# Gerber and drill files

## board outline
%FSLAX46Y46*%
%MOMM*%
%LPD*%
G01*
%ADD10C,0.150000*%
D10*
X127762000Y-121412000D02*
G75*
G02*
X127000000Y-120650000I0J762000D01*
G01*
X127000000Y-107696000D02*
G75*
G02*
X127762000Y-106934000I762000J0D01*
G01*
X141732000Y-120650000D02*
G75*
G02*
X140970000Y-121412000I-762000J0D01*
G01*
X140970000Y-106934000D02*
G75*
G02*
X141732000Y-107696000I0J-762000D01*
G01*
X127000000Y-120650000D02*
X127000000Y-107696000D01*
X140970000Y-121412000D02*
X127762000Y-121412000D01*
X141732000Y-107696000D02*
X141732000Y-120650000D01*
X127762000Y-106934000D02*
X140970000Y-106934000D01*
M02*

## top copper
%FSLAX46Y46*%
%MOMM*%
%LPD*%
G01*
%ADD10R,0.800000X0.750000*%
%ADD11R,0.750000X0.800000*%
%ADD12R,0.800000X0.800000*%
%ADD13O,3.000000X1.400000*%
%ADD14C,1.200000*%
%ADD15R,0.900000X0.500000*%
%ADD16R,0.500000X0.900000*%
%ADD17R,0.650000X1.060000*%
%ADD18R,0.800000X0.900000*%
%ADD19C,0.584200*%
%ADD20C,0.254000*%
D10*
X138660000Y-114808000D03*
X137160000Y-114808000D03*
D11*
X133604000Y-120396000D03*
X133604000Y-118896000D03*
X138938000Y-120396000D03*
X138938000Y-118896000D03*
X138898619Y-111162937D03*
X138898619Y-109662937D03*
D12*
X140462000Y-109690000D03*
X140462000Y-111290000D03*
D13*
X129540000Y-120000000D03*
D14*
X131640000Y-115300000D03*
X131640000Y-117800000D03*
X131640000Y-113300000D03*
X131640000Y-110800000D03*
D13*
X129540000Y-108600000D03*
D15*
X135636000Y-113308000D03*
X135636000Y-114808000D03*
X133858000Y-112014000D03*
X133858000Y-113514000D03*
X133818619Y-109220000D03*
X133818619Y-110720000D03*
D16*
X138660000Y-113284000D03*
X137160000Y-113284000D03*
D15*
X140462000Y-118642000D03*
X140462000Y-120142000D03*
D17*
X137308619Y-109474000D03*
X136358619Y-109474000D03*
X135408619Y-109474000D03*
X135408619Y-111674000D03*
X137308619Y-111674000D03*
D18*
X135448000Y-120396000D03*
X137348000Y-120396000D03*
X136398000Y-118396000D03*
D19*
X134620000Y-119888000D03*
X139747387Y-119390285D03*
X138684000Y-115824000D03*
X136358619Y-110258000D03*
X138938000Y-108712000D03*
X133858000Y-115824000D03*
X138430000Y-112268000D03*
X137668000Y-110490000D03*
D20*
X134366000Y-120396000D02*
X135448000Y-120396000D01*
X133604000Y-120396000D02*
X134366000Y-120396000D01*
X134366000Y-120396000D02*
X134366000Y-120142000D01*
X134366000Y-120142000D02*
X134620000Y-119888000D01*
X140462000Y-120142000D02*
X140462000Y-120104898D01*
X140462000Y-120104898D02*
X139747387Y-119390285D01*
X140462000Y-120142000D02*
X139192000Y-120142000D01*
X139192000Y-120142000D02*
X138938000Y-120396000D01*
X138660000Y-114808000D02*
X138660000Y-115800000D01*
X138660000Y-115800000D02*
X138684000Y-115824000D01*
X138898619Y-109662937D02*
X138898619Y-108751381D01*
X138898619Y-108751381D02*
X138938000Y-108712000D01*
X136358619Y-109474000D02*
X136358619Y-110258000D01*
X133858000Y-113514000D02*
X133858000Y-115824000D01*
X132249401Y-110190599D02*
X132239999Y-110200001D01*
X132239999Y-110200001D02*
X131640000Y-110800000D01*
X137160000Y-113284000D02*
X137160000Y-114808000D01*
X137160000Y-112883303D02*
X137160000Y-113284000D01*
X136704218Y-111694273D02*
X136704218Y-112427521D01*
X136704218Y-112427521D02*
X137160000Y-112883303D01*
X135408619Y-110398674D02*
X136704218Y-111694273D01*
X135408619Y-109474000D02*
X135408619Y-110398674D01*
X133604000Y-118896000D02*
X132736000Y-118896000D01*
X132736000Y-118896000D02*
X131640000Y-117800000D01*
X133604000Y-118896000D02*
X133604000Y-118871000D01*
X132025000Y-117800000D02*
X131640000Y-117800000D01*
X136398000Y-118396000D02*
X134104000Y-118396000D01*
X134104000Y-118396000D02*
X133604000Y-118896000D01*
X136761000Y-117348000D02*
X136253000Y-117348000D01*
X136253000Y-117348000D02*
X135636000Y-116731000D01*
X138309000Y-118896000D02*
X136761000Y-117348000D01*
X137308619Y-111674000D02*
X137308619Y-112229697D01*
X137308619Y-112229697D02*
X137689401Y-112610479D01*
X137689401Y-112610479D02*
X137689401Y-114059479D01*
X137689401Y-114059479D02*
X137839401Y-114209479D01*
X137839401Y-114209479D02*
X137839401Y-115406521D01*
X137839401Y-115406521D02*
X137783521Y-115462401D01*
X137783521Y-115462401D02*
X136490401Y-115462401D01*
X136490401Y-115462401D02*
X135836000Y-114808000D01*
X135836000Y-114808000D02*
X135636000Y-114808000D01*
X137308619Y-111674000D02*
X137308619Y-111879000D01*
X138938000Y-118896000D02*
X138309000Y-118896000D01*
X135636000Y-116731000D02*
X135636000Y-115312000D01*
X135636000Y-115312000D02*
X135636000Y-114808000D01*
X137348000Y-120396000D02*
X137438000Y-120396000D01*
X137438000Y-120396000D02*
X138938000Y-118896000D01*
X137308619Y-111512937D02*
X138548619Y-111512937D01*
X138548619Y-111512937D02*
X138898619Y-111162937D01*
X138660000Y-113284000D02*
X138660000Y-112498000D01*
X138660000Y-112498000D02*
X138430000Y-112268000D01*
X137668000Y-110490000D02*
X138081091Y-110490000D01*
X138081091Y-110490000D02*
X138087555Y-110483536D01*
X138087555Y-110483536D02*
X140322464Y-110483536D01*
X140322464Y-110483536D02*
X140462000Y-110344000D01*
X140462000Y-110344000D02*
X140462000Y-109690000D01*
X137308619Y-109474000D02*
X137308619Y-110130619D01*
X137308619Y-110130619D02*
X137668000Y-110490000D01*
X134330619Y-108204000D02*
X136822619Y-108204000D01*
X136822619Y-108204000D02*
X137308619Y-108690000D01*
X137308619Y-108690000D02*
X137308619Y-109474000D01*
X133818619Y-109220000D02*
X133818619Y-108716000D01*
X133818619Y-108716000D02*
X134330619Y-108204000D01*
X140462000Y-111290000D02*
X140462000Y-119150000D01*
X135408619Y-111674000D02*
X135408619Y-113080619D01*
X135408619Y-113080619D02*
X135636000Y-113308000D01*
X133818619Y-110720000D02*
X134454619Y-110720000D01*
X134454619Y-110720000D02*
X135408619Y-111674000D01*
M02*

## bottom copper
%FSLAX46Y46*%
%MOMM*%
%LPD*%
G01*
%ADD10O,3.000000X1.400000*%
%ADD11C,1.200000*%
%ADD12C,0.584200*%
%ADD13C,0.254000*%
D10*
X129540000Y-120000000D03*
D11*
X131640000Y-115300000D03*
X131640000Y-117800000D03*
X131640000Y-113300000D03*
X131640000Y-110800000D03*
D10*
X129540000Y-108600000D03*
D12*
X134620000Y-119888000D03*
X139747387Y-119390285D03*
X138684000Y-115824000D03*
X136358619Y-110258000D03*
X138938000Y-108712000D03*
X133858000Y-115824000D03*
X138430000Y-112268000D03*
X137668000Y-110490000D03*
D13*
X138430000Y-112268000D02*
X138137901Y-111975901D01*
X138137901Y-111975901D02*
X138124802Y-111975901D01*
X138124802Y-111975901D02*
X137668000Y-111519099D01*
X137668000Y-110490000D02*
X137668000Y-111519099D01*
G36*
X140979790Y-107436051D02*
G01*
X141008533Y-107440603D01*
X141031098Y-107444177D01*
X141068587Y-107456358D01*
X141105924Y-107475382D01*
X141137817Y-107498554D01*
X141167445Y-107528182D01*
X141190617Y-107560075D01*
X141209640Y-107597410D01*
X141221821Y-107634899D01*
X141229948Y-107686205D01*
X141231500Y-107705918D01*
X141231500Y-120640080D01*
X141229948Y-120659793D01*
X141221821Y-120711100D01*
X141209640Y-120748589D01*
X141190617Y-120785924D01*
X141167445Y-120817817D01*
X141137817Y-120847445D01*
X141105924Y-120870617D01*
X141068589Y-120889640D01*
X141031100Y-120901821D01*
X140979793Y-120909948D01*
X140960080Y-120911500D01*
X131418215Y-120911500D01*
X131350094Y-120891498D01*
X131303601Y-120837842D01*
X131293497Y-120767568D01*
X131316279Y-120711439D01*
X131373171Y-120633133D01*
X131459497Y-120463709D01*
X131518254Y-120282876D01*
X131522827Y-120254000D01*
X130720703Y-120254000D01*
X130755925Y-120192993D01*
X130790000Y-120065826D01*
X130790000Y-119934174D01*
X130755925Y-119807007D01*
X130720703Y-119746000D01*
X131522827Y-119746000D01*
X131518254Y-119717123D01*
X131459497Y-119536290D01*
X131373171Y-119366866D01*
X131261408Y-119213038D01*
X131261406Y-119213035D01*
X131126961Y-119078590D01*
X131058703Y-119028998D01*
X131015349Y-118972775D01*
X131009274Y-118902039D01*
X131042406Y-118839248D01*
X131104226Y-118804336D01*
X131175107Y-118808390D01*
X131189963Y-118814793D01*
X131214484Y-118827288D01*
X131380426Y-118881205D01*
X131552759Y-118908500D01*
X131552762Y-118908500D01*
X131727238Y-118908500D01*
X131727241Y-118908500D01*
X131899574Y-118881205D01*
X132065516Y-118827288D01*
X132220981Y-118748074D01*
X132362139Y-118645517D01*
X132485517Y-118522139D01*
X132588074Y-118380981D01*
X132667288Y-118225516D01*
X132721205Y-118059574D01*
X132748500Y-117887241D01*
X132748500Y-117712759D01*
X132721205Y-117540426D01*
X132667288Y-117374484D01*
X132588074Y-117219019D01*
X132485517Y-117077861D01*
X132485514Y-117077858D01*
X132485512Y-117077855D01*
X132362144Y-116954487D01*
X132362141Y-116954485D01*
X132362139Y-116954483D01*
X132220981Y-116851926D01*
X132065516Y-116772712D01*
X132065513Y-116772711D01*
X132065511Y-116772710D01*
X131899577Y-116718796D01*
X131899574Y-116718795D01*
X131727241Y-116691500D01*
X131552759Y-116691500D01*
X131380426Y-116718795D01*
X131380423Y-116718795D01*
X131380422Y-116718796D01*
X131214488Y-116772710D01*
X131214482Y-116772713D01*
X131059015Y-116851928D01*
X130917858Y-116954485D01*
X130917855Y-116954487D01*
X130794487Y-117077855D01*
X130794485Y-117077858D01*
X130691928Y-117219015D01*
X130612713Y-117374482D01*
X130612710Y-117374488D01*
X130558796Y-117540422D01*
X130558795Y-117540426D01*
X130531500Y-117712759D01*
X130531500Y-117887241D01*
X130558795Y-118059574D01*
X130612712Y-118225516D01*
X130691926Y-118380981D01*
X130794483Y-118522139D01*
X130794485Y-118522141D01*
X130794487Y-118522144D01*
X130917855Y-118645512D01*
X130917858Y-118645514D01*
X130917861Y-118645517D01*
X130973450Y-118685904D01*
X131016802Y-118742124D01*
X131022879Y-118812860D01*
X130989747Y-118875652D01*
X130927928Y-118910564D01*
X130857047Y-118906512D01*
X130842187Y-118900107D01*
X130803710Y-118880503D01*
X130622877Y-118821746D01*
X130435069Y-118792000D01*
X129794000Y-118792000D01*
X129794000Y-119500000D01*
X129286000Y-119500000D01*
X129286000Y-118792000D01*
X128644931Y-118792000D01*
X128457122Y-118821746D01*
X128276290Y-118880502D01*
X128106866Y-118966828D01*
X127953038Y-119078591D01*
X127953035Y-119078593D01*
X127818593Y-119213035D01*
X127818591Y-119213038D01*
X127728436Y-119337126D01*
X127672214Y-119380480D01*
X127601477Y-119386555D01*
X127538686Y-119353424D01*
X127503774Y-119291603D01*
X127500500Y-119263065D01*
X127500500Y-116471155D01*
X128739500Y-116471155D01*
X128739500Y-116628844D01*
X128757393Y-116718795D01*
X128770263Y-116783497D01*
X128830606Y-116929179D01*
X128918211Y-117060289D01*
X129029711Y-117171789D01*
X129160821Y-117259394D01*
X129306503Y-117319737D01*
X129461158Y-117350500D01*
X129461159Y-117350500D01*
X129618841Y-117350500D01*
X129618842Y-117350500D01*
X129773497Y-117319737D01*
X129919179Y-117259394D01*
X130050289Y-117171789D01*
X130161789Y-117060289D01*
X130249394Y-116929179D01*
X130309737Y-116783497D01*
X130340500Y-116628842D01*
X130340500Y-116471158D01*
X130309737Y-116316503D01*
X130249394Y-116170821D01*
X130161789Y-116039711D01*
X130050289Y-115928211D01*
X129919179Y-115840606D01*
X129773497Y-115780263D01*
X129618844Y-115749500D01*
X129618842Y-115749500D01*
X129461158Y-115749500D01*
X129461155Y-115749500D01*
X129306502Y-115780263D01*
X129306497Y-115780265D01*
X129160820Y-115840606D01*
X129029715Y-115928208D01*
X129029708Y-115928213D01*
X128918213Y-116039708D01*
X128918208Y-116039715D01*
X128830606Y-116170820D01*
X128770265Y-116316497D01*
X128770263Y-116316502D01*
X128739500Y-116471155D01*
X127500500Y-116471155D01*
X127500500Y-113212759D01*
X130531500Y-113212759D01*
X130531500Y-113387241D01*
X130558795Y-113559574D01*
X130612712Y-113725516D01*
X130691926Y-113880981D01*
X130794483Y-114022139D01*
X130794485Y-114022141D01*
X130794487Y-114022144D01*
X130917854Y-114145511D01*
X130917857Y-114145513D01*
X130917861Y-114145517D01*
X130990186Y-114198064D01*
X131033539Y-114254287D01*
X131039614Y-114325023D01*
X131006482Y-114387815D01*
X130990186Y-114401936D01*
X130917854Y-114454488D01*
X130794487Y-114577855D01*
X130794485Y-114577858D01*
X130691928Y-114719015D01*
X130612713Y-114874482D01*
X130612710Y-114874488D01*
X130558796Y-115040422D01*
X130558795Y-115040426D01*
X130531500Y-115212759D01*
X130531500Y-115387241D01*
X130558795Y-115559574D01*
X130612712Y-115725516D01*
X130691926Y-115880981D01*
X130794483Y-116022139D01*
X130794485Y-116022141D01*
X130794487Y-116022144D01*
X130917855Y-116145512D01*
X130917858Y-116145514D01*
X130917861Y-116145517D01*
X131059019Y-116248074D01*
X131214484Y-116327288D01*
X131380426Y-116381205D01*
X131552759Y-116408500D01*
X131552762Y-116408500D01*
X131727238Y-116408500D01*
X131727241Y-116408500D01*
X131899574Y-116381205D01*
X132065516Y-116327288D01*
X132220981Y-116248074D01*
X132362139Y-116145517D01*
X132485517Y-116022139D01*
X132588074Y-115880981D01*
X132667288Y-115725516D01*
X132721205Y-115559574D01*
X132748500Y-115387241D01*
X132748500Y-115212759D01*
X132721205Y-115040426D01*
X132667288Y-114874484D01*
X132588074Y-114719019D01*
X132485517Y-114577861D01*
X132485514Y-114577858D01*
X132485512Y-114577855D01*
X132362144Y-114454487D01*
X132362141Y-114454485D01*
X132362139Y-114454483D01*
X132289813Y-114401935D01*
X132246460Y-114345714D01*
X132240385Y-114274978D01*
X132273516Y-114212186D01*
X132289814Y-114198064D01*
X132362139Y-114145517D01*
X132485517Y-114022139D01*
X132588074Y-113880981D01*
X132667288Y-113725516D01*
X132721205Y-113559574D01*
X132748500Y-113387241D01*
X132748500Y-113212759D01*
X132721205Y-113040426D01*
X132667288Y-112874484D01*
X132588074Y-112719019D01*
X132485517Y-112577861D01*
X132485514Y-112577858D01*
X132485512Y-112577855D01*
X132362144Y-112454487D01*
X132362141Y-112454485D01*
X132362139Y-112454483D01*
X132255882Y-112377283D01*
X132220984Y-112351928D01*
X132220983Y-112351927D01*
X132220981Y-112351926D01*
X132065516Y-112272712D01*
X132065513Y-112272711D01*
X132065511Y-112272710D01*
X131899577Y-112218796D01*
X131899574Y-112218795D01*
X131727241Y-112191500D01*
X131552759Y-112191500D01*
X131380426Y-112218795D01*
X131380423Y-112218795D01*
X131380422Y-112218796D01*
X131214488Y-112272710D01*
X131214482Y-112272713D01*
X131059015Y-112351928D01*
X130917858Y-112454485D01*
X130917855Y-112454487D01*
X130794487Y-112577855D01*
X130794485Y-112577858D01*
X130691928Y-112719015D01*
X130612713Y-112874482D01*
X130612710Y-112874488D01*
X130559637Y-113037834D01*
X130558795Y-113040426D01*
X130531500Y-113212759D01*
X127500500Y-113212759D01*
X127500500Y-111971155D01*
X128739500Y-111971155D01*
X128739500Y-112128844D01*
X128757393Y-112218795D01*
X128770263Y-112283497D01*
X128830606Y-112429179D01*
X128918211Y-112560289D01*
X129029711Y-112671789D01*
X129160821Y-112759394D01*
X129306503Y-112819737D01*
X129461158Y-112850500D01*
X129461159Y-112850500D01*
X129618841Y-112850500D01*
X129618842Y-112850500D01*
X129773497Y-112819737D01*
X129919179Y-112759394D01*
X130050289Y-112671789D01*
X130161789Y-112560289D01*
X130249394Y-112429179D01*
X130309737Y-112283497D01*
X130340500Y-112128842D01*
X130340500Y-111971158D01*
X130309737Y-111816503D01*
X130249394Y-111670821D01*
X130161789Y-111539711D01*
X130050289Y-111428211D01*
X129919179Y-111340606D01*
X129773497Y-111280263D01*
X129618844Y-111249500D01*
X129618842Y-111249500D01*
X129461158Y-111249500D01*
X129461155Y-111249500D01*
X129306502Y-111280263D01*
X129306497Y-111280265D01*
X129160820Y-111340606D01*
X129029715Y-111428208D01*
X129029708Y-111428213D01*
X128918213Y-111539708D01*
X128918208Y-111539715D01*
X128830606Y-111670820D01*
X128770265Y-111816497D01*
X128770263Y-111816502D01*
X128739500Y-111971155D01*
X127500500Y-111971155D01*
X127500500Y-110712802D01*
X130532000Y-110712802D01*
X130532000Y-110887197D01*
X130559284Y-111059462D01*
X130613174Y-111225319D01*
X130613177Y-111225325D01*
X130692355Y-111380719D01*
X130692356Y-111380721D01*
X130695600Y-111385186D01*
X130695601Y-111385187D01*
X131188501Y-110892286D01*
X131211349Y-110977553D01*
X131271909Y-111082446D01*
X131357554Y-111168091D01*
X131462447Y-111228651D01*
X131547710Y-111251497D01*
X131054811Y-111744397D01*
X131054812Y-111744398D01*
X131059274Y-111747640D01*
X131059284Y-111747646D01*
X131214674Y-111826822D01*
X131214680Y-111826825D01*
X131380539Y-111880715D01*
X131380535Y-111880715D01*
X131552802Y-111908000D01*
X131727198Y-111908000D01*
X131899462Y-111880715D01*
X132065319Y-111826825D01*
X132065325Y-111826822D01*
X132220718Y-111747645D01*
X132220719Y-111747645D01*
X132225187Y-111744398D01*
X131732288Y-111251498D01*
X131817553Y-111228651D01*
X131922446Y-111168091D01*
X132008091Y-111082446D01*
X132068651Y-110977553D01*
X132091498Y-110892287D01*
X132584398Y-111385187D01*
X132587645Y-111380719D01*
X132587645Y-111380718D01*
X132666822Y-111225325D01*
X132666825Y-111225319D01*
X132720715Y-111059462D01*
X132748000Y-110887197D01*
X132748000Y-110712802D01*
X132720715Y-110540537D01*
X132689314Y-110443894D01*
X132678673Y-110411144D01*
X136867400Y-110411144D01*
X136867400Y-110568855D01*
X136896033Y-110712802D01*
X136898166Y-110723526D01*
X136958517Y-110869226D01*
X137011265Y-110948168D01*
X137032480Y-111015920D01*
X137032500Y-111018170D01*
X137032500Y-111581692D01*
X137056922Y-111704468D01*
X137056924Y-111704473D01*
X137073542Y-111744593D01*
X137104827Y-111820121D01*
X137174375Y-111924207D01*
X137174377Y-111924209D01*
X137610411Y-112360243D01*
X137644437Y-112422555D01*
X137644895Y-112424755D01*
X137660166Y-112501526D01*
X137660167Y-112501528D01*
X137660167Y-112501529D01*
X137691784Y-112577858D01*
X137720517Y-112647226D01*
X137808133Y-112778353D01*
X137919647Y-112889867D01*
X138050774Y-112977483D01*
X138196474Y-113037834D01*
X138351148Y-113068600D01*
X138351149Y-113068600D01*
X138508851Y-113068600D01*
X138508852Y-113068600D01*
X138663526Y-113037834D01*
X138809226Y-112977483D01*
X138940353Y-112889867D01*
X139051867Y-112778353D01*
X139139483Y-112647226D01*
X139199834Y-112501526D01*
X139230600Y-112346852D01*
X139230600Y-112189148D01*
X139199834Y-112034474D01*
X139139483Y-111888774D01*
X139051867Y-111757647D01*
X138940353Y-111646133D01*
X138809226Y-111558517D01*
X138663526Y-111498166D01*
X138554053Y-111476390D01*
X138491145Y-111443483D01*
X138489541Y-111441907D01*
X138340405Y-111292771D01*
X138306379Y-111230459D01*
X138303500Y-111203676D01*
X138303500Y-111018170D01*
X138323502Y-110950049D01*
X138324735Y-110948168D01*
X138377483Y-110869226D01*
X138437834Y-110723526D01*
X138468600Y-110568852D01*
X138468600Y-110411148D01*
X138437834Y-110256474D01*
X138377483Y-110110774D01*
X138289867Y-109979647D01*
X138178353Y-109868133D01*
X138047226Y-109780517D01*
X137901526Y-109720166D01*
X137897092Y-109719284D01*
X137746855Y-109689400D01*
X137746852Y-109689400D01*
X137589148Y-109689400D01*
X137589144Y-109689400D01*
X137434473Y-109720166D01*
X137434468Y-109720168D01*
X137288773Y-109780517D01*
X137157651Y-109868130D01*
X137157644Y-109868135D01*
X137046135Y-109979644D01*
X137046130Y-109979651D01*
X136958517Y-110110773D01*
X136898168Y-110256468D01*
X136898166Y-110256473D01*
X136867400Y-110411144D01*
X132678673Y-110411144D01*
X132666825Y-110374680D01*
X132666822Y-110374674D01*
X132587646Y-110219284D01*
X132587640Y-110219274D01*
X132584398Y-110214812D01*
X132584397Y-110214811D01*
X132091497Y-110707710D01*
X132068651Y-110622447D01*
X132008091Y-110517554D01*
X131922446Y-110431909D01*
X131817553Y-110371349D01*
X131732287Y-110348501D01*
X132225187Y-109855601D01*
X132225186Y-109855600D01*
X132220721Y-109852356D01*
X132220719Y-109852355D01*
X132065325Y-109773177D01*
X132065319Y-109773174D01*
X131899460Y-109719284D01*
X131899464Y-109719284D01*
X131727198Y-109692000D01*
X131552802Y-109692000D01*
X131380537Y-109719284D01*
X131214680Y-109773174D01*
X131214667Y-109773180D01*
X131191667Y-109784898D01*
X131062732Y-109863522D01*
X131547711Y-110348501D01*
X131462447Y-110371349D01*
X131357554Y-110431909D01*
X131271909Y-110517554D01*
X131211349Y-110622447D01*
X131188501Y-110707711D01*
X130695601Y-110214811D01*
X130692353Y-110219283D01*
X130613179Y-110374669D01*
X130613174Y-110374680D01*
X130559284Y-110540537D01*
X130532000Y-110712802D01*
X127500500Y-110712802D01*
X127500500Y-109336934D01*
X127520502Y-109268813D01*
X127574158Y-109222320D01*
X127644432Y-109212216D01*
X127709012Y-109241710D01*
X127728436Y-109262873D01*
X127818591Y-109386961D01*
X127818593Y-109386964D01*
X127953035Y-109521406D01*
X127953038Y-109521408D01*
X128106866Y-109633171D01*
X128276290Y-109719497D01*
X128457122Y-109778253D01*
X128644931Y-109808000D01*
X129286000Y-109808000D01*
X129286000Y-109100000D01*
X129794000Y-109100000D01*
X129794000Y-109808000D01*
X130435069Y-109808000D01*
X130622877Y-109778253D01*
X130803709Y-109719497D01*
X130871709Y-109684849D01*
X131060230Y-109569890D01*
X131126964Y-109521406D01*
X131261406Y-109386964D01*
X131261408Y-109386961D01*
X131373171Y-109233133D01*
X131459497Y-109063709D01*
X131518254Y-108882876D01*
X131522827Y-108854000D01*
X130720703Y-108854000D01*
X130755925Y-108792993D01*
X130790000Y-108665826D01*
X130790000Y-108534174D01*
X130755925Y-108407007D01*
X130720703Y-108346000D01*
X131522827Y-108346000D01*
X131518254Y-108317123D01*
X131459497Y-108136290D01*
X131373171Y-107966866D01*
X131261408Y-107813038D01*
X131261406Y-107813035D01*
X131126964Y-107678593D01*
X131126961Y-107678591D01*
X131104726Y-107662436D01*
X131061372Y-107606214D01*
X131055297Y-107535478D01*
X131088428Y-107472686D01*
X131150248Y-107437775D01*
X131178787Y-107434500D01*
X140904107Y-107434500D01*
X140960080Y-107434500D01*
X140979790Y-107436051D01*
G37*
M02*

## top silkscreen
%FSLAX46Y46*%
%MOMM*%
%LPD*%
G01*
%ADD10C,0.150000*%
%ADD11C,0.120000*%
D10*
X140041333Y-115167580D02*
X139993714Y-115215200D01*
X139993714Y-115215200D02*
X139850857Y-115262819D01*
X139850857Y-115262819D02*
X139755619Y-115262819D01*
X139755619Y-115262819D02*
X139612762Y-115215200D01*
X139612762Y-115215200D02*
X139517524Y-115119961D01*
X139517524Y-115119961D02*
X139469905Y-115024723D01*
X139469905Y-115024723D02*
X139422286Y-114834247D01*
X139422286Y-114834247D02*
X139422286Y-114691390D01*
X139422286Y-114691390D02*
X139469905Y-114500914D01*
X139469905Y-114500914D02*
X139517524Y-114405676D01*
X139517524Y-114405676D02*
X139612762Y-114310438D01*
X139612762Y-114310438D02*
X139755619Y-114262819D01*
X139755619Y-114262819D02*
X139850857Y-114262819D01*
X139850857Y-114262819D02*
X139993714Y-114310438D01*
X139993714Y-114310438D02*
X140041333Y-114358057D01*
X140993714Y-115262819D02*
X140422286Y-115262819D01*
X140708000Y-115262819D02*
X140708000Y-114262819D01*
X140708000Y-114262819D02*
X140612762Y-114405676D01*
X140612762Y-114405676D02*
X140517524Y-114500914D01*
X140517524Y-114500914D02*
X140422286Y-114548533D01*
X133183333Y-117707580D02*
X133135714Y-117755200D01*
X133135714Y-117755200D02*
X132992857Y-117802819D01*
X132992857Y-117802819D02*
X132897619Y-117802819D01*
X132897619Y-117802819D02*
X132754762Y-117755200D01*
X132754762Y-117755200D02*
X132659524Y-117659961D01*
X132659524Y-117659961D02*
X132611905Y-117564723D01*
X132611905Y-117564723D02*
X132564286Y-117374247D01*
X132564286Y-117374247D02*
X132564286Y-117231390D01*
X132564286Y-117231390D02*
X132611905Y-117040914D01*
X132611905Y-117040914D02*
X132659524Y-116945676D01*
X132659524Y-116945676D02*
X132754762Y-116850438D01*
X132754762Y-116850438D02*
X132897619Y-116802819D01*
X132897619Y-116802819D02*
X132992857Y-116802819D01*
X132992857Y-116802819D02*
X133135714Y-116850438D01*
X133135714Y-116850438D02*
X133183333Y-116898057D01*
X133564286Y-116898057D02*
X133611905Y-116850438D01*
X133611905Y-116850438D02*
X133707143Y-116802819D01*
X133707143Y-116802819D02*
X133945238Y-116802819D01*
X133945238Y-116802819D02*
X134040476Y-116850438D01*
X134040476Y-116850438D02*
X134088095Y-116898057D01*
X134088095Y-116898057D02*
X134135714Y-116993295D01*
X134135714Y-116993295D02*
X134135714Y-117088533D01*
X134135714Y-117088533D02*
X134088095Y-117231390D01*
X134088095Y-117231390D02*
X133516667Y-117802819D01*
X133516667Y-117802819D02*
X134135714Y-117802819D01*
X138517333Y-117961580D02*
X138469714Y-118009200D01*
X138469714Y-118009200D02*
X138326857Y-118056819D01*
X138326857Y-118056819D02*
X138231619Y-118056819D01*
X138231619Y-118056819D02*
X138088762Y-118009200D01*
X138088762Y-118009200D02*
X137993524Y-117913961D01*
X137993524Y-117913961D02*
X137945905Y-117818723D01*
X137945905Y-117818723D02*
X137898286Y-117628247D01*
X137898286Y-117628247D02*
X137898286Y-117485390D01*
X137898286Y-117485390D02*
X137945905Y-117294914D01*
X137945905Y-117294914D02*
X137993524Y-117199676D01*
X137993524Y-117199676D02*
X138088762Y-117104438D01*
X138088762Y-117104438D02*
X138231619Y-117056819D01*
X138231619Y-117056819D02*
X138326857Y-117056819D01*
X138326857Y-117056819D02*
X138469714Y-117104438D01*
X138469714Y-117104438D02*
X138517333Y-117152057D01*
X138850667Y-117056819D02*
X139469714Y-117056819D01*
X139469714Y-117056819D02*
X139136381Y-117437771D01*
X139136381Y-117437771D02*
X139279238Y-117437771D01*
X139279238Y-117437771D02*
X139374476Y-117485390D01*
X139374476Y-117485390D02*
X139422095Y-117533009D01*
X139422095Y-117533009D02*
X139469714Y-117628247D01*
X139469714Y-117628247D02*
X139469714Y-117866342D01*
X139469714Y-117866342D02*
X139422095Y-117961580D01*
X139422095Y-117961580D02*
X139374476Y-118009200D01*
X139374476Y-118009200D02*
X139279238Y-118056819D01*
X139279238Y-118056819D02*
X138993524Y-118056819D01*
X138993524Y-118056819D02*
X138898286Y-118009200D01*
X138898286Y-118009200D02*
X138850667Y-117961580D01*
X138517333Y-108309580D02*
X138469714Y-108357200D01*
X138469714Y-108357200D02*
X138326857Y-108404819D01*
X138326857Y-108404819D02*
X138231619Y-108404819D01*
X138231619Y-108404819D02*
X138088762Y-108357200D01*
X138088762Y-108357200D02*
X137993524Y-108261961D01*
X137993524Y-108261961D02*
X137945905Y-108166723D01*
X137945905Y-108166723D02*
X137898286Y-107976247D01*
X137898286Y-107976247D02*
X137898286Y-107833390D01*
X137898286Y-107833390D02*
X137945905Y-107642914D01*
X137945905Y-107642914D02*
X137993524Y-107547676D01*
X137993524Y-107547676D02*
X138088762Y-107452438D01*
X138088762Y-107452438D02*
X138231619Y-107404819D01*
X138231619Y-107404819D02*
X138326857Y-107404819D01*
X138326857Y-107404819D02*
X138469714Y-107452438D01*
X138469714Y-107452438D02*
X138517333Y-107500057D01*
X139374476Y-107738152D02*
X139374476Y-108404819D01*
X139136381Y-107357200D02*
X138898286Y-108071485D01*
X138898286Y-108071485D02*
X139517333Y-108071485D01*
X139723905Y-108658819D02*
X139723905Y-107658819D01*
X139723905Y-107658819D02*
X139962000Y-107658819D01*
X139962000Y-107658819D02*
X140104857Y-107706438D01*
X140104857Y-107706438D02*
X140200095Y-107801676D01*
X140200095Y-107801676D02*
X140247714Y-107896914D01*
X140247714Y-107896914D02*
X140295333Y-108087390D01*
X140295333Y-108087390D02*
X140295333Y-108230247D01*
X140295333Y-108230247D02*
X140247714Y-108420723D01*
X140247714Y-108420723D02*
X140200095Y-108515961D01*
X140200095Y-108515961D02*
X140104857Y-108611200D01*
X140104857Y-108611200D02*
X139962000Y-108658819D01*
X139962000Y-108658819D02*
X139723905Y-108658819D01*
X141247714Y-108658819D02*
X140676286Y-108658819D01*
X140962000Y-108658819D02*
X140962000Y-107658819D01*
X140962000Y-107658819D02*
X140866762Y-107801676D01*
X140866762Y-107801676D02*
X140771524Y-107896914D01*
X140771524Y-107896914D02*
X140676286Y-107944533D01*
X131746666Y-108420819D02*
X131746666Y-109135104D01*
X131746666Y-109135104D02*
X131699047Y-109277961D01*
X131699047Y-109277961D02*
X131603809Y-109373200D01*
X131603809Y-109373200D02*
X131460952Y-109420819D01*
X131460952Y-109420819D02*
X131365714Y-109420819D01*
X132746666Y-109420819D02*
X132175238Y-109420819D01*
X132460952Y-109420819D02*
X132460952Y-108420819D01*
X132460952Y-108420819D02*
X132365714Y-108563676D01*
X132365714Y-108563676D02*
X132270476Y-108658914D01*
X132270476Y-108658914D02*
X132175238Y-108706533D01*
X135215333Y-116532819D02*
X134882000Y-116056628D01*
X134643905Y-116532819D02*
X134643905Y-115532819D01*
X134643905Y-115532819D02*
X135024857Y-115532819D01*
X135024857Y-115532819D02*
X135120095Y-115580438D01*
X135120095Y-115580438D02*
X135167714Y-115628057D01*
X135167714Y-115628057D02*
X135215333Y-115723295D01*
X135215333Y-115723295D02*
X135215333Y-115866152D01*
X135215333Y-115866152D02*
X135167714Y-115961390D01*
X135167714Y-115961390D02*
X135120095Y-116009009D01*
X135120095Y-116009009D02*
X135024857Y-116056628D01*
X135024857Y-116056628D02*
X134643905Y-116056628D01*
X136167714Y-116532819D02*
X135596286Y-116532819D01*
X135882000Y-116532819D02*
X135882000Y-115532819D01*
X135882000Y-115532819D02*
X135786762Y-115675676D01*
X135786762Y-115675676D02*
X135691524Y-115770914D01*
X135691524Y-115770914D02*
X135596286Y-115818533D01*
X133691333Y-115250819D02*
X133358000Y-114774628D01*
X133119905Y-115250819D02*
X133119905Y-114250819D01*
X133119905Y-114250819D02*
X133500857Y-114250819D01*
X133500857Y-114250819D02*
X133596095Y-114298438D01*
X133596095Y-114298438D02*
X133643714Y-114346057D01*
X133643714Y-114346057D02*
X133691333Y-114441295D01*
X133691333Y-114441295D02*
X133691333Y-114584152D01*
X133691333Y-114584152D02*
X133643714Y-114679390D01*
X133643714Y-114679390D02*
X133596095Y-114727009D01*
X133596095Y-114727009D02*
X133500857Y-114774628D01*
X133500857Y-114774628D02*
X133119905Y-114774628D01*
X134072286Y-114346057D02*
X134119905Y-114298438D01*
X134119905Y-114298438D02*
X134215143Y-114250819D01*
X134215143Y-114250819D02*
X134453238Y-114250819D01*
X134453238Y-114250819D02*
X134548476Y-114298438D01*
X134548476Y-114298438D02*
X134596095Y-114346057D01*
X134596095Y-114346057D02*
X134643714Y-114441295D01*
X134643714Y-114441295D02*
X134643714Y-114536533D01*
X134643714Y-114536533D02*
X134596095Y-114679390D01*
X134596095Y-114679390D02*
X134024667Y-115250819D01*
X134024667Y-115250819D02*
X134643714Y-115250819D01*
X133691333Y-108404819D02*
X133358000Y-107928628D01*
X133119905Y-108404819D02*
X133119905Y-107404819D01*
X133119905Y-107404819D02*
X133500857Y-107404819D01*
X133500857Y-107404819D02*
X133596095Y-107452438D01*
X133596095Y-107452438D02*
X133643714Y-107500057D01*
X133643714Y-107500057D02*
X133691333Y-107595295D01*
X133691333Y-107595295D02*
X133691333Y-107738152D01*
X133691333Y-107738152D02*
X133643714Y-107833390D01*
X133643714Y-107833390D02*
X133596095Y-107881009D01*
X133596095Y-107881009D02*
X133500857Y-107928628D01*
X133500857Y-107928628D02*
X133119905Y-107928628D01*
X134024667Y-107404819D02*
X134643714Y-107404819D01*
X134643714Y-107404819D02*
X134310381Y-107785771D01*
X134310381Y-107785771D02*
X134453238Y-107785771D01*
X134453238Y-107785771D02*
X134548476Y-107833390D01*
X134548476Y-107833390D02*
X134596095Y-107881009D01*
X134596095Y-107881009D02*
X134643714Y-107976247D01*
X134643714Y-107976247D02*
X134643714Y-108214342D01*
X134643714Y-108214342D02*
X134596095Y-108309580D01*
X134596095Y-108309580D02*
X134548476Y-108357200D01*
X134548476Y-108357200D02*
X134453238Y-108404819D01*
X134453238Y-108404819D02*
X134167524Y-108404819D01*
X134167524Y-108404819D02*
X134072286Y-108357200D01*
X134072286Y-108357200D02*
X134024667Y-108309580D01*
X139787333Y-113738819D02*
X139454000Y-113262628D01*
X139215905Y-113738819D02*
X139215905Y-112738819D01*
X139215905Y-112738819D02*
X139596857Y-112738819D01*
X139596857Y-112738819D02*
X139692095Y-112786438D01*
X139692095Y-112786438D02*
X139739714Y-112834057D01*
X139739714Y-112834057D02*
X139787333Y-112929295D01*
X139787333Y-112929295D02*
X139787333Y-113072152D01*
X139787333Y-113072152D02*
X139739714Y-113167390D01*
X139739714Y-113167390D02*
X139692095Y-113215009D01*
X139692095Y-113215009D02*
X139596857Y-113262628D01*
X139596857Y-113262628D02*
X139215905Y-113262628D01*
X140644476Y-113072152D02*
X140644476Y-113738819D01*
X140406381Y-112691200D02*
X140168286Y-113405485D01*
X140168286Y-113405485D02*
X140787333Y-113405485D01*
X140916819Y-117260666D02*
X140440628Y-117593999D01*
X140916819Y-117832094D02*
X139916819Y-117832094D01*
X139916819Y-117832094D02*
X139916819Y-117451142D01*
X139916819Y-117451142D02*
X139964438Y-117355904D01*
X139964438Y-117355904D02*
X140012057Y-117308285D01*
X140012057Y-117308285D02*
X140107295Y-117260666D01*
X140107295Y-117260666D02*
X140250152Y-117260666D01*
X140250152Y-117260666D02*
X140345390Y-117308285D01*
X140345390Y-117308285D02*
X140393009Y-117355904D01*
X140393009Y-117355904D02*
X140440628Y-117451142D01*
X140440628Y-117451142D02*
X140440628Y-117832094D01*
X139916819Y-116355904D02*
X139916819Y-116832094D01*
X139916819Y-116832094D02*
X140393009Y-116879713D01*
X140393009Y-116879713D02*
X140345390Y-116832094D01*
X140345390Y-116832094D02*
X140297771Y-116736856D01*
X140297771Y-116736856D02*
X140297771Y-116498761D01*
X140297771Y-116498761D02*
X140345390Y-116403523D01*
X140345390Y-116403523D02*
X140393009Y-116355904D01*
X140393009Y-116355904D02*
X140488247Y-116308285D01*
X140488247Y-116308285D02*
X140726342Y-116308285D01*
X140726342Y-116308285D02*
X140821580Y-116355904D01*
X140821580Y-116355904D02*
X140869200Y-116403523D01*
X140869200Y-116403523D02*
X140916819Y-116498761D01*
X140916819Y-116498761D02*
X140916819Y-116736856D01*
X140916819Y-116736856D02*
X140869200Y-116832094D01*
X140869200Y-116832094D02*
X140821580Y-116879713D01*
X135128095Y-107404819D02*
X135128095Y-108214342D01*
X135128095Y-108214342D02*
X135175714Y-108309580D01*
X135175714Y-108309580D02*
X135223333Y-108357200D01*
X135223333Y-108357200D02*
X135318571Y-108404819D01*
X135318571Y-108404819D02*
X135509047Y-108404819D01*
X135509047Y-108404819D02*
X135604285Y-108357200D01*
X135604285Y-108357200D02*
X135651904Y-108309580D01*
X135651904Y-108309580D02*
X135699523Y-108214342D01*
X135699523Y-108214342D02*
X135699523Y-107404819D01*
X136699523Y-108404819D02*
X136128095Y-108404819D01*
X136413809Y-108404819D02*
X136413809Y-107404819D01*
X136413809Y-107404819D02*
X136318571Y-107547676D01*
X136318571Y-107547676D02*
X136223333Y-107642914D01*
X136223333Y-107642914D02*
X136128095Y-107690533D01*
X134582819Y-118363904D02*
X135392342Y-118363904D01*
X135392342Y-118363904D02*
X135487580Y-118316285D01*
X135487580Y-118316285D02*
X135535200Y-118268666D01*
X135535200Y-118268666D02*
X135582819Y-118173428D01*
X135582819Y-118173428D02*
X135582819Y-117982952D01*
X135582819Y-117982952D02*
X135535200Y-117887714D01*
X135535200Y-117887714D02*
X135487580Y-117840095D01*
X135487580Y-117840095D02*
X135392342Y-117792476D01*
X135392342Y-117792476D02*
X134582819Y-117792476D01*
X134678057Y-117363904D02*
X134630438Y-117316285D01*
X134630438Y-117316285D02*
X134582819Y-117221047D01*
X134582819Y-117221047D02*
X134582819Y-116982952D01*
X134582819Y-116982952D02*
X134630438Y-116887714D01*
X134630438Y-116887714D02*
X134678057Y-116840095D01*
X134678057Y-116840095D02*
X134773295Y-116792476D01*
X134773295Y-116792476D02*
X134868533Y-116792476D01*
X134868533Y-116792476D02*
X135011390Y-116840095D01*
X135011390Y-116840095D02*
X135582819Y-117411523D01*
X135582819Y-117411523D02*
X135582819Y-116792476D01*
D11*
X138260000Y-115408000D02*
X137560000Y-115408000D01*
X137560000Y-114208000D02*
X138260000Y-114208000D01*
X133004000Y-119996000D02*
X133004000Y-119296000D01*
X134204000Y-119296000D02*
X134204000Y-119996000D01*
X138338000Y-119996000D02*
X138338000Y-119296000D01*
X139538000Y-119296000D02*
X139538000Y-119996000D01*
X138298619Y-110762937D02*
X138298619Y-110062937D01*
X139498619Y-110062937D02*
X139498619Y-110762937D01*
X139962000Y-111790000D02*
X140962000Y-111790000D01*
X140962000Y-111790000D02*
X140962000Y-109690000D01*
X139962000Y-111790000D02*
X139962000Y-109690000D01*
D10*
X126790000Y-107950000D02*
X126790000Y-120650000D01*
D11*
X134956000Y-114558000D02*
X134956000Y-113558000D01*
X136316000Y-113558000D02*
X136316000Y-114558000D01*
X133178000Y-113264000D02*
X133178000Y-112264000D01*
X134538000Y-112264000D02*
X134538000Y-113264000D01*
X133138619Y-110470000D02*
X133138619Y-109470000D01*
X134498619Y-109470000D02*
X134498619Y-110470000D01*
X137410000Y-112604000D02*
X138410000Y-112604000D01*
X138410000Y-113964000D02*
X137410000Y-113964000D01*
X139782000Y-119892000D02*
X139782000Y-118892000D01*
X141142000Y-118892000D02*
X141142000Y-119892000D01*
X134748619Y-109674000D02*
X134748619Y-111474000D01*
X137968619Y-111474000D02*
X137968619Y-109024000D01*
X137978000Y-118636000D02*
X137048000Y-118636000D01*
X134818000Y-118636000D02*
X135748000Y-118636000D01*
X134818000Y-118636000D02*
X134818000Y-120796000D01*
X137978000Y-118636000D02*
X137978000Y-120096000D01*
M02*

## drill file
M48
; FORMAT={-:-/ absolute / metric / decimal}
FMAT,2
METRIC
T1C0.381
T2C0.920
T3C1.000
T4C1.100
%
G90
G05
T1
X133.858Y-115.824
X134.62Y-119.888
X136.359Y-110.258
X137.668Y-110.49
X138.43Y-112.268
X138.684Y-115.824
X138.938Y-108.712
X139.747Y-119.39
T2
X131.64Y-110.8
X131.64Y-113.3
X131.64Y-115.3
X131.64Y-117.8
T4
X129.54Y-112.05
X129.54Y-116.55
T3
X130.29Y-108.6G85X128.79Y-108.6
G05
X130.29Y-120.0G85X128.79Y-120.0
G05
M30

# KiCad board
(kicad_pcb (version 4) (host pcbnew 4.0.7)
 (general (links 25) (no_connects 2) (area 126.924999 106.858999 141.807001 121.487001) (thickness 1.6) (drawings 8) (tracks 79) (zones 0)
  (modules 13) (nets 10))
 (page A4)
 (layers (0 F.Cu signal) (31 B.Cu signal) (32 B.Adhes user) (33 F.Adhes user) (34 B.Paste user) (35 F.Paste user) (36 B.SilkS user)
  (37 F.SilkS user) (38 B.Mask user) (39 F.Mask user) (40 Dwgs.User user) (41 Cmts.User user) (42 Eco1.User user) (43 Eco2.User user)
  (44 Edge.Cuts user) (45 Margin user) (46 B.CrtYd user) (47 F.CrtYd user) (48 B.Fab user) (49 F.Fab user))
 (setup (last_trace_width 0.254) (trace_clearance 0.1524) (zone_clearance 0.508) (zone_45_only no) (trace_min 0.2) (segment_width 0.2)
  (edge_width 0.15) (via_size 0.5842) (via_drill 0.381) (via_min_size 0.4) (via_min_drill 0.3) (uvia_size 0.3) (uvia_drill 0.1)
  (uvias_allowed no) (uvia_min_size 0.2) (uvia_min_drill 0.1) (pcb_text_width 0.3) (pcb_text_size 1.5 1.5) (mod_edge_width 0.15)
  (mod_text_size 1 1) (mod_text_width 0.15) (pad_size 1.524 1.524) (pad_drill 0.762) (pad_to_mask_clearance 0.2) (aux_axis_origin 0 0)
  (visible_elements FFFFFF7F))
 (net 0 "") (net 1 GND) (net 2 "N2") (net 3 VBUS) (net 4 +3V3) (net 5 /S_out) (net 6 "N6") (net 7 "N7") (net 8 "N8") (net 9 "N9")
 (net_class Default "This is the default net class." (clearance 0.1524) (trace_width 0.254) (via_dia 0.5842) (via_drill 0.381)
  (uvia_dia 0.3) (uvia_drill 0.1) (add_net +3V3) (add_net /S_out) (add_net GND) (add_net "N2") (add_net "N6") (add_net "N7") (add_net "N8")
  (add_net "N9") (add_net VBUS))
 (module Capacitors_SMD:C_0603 (layer F.Cu) (at 137.91 114.808)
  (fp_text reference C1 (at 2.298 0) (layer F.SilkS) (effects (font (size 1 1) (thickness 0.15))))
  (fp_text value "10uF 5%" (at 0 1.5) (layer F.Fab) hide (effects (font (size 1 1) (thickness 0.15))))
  (fp_line (start 0.35 0.6) (end -0.35 0.6) (layer F.SilkS) (width 0.12))
  (fp_line (start -0.35 -0.6) (end 0.35 -0.6) (layer F.SilkS) (width 0.12))
  (pad 2 smd rect (at 0.75 0) (size 0.8 0.75) (layers F.Cu F.Paste F.Mask) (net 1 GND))
  (pad 1 smd rect (at -0.75 0) (size 0.8 0.75) (layers F.Cu F.Paste F.Mask) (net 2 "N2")))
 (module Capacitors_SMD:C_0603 (layer F.Cu) (at 133.604 119.646 270)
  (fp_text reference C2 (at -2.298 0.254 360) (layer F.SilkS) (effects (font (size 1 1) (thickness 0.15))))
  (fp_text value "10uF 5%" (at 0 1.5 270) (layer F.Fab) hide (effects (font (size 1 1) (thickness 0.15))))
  (fp_line (start 0.35 0.6) (end -0.35 0.6) (layer F.SilkS) (width 0.12))
  (fp_line (start -0.35 -0.6) (end 0.35 -0.6) (layer F.SilkS) (width 0.12))
  (pad 2 smd rect (at 0.75 0 270) (size 0.8 0.75) (layers F.Cu F.Paste F.Mask) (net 1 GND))
  (pad 1 smd rect (at -0.75 0 270) (size 0.8 0.75) (layers F.Cu F.Paste F.Mask) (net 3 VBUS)))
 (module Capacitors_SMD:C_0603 (layer F.Cu) (at 138.938 119.646 270)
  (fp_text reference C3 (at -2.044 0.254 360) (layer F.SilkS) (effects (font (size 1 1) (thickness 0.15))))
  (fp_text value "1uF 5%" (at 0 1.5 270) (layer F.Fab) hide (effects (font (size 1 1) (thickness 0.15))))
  (fp_line (start 0.35 0.6) (end -0.35 0.6) (layer F.SilkS) (width 0.12))
  (fp_line (start -0.35 -0.6) (end 0.35 -0.6) (layer F.SilkS) (width 0.12))
  (pad 2 smd rect (at 0.75 0 270) (size 0.8 0.75) (layers F.Cu F.Paste F.Mask) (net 1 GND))
  (pad 1 smd rect (at -0.75 0 270) (size 0.8 0.75) (layers F.Cu F.Paste F.Mask) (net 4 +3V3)))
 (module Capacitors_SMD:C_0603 (layer F.Cu) (at 138.898619 110.412937 270)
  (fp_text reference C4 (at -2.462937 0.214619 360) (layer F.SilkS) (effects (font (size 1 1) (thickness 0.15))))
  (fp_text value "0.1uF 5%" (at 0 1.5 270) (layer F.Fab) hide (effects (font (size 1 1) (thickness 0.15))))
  (fp_line (start 0.35 0.6) (end -0.35 0.6) (layer F.SilkS) (width 0.12))
  (fp_line (start -0.35 -0.6) (end 0.35 -0.6) (layer F.SilkS) (width 0.12))
  (pad 2 smd rect (at 0.75 0 270) (size 0.8 0.75) (layers F.Cu F.Paste F.Mask) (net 4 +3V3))
  (pad 1 smd rect (at -0.75 0 270) (size 0.8 0.75) (layers F.Cu F.Paste F.Mask) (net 1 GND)))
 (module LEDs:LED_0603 (layer F.Cu) (at 140.462 110.49 90)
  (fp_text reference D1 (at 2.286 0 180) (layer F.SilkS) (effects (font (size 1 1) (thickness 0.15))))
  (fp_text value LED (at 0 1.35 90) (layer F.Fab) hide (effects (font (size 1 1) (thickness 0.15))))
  (fp_line (start -1.3 -0.5) (end -1.3 0.5) (layer F.SilkS) (width 0.12))
  (fp_line (start -1.3 0.5) (end 0.8 0.5) (layer F.SilkS) (width 0.12))
  (fp_line (start -1.3 -0.5) (end 0.8 -0.5) (layer F.SilkS) (width 0.12))
  (pad 2 smd rect (at 0.8 0 270) (size 0.8 0.8) (layers F.Cu F.Paste F.Mask) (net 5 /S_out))
  (pad 1 smd rect (at -0.8 0 270) (size 0.8 0.8) (layers F.Cu F.Paste F.Mask) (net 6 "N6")))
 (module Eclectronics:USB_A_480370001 (layer F.Cu) (at 129.54 114.3 270)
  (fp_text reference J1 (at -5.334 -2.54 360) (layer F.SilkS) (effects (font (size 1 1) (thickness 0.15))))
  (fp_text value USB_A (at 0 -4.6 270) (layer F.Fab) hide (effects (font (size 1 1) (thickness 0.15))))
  (fp_line (start -6.35 2.75) (end 6.35 2.75) (layer F.SilkS) (width 0.15))
  (pad 5 thru_hole oval (at 5.7 0 270) (size 1.4 3) (drill oval 1 2.5) (layers *.Cu *.Mask) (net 1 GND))
  (pad 2 thru_hole circle (at 1 -2.1 270) (size 1.2 1.2) (drill 0.92) (layers *.Cu *.Mask) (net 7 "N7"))
  (pad 1 thru_hole circle (at 3.5 -2.1 270) (size 1.2 1.2) (drill 0.92) (layers *.Cu *.Mask) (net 3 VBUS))
  (pad 3 thru_hole circle (at -1 -2.1 270) (size 1.2 1.2) (drill 0.92) (layers *.Cu *.Mask) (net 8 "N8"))
  (pad 4 thru_hole circle (at -3.5 -2.1 270) (size 1.2 1.2) (drill 0.92) (layers *.Cu *.Mask) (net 1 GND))
  (pad "" np_thru_hole circle (at 2.25 0 270) (size 1.1 1.1) (drill 1.1) (layers *.Cu *.Mask))
  (pad "" np_thru_hole circle (at -2.25 0 270) (size 1.1 1.1) (drill 1.1) (layers *.Cu *.Mask))
  (pad 5 thru_hole oval (at -5.7 0 270) (size 1.4 3) (drill oval 1 2.5) (layers *.Cu *.Mask) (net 1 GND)))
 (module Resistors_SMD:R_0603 (layer F.Cu) (at 135.636 114.058 270)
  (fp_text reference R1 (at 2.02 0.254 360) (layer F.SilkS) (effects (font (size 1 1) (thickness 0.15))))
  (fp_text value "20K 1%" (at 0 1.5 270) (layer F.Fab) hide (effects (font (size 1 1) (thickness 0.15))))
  (fp_line (start 0.5 0.68) (end -0.5 0.68) (layer F.SilkS) (width 0.12))
  (fp_line (start -0.5 -0.68) (end 0.5 -0.68) (layer F.SilkS) (width 0.12))
  (pad 1 smd rect (at -0.75 0 270) (size 0.5 0.9) (layers F.Cu F.Paste F.Mask) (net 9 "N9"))
  (pad 2 smd rect (at 0.75 0 270) (size 0.5 0.9) (layers F.Cu F.Paste F.Mask) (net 4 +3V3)))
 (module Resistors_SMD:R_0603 (layer F.Cu) (at 133.858 112.764 270)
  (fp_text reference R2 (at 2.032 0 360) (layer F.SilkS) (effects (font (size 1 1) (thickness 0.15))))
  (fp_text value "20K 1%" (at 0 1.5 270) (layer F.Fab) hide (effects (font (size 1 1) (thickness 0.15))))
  (fp_line (start 0.5 0.68) (end -0.5 0.68) (layer F.SilkS) (width 0.12))
  (fp_line (start -0.5 -0.68) (end 0.5 -0.68) (layer F.SilkS) (width 0.12))
  (pad 1 smd rect (at -0.75 0 270) (size 0.5 0.9) (layers F.Cu F.Paste F.Mask) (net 9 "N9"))
  (pad 2 smd rect (at 0.75 0 270) (size 0.5 0.9) (layers F.Cu F.Paste F.Mask) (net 1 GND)))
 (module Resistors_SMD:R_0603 (layer F.Cu) (at 133.818619 109.97 270)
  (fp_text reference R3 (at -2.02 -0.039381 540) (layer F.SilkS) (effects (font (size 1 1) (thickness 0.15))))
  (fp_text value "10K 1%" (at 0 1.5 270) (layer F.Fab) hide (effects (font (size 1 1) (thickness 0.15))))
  (fp_line (start 0.5 0.68) (end -0.5 0.68) (layer F.SilkS) (width 0.12))
  (fp_line (start -0.5 -0.68) (end 0.5 -0.68) (layer F.SilkS) (width 0.12))
  (pad 1 smd rect (at -0.75 0 270) (size 0.5 0.9) (layers F.Cu F.Paste F.Mask) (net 5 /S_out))
  (pad 2 smd rect (at 0.75 0 270) (size 0.5 0.9) (layers F.Cu F.Paste F.Mask) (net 9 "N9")))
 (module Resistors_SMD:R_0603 (layer F.Cu) (at 137.91 113.284 180)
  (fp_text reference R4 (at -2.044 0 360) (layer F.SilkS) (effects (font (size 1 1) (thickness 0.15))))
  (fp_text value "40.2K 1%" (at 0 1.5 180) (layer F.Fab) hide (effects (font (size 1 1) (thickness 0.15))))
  (fp_line (start 0.5 0.68) (end -0.5 0.68) (layer F.SilkS) (width 0.12))
  (fp_line (start -0.5 -0.68) (end 0.5 -0.68) (layer F.SilkS) (width 0.12))
  (pad 1 smd rect (at -0.75 0 180) (size 0.5 0.9) (layers F.Cu F.Paste F.Mask) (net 5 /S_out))
  (pad 2 smd rect (at 0.75 0 180) (size 0.5 0.9) (layers F.Cu F.Paste F.Mask) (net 2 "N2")))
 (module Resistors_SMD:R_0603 (layer F.Cu) (at 140.462 119.392 270)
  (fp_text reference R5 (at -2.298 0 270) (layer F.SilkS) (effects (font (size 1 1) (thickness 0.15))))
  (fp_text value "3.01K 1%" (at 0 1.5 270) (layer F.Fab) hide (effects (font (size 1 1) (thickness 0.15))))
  (fp_line (start 0.5 0.68) (end -0.5 0.68) (layer F.SilkS) (width 0.12))
  (fp_line (start -0.5 -0.68) (end 0.5 -0.68) (layer F.SilkS) (width 0.12))
  (pad 1 smd rect (at -0.75 0 270) (size 0.5 0.9) (layers F.Cu F.Paste F.Mask) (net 6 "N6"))
  (pad 2 smd rect (at 0.75 0 270) (size 0.5 0.9) (layers F.Cu F.Paste F.Mask) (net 1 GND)))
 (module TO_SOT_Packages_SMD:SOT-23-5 (layer F.Cu) (at 136.358619 110.574 270)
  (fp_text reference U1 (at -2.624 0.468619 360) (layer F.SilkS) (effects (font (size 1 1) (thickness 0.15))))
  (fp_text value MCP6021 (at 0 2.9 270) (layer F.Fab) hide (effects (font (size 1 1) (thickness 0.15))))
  (fp_line (start -0.9 1.61) (end 0.9 1.61) (layer F.SilkS) (width 0.12))
  (fp_line (start 0.9 -1.61) (end -1.55 -1.61) (layer F.SilkS) (width 0.12))
  (pad 1 smd rect (at -1.1 -0.95 270) (size 1.06 0.65) (layers F.Cu F.Paste F.Mask) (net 5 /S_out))
  (pad 2 smd rect (at -1.1 0 270) (size 1.06 0.65) (layers F.Cu F.Paste F.Mask) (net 1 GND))
  (pad 3 smd rect (at -1.1 0.95 270) (size 1.06 0.65) (layers F.Cu F.Paste F.Mask) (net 2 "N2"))
  (pad 4 smd rect (at 1.1 0.95 270) (size 1.06 0.65) (layers F.Cu F.Paste F.Mask) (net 9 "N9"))
  (pad 5 smd rect (at 1.1 -0.95 270) (size 1.06 0.65) (layers F.Cu F.Paste F.Mask) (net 4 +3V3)))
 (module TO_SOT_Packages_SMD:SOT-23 (layer F.Cu) (at 136.398 119.396 90)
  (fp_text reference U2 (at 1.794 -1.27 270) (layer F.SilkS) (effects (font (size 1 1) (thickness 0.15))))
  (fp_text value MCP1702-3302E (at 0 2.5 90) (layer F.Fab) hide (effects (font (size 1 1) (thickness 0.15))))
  (fp_line (start 0.76 1.58) (end 0.76 0.65) (layer F.SilkS) (width 0.12))
  (fp_line (start 0.76 -1.58) (end 0.76 -0.65) (layer F.SilkS) (width 0.12))
  (fp_line (start 0.76 -1.58) (end -1.4 -1.58) (layer F.SilkS) (width 0.12))
  (fp_line (start 0.76 1.58) (end -0.7 1.58) (layer F.SilkS) (width 0.12))
  (pad 1 smd rect (at -1 -0.95 90) (size 0.9 0.8) (layers F.Cu F.Paste F.Mask) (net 1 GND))
  (pad 2 smd rect (at -1 0.95 90) (size 0.9 0.8) (layers F.Cu F.Paste F.Mask) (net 4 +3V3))
  (pad 3 smd rect (at 1 0 90) (size 0.9 0.8) (layers F.Cu F.Paste F.Mask) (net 3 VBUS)))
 (gr_arc (start 127.762 120.65) (end 127.762 121.412) (angle 90) (layer Edge.Cuts) (width 0.15))
 (gr_arc (start 127.762 107.696) (end 127 107.696) (angle 90) (layer Edge.Cuts) (width 0.15))
 (gr_arc (start 140.97 120.65) (end 141.732 120.65) (angle 90) (layer Edge.Cuts) (width 0.15))
 (gr_arc (start 140.97 107.696) (end 140.97 106.934) (angle 90) (layer Edge.Cuts) (width 0.15))
 (gr_line (start 127 120.65) (end 127 107.696) (layer Edge.Cuts) (width 0.15))
 (gr_line (start 140.97 121.412) (end 127.762 121.412) (layer Edge.Cuts) (width 0.15))
 (gr_line (start 141.732 107.696) (end 141.732 120.65) (layer Edge.Cuts) (width 0.15))
 (gr_line (start 127.762 106.934) (end 140.97 106.934) (layer Edge.Cuts) (width 0.15))
 (segment (start 134.366 120.396) (end 135.448 120.396) (width 0.254) (layer F.Cu) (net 1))
 (segment (start 133.604 120.396) (end 134.366 120.396) (width 0.254) (layer F.Cu) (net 1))
 (via (at 134.62 119.888) (size 0.5842) (drill 0.381) (layers F.Cu B.Cu) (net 1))
 (segment (start 134.366 120.396) (end 134.366 120.142) (width 0.254) (layer F.Cu) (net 1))
 (segment (start 134.366 120.142) (end 134.62 119.888) (width 0.254) (layer F.Cu) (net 1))
 (segment (start 140.462 120.142) (end 140.462 120.104898) (width 0.254) (layer F.Cu) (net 1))
 (segment (start 140.462 120.104898) (end 139.747387 119.390285) (width 0.254) (layer F.Cu) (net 1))
 (via (at 139.747387 119.390285) (size 0.5842) (drill 0.381) (layers F.Cu B.Cu) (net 1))
 (segment (start 140.462 120.142) (end 139.192 120.142) (width 0.254) (layer F.Cu) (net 1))
 (segment (start 139.192 120.142) (end 138.938 120.396) (width 0.254) (layer F.Cu) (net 1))
 (segment (start 138.66 114.808) (end 138.66 115.8) (width 0.254) (layer F.Cu) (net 1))
 (segment (start 138.66 115.8) (end 138.684 115.824) (width 0.254) (layer F.Cu) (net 1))
 (via (at 138.684 115.824) (size 0.5842) (drill 0.381) (layers F.Cu B.Cu) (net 1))
 (via (at 136.358619 110.258) (size 0.5842) (drill 0.381) (layers F.Cu B.Cu) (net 1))
 (segment (start 138.898619 109.662937) (end 138.898619 108.751381) (width 0.254) (layer F.Cu) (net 1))
 (segment (start 138.898619 108.751381) (end 138.938 108.712) (width 0.254) (layer F.Cu) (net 1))
 (via (at 138.938 108.712) (size 0.5842) (drill 0.381) (layers F.Cu B.Cu) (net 1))
 (segment (start 136.358619 109.474) (end 136.358619 110.258) (width 0.254) (layer F.Cu) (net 1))
 (segment (start 133.858 113.514) (end 133.858 115.824) (width 0.254) (layer F.Cu) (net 1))
 (via (at 133.858 115.824) (size 0.5842) (drill 0.381) (layers F.Cu B.Cu) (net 1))
 (segment (start 132.249401 110.190599) (end 132.239999 110.200001) (width 0.254) (layer F.Cu) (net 1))
 (segment (start 132.239999 110.200001) (end 131.64 110.8) (width 0.254) (layer F.Cu) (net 1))
 (segment (start 137.16 113.284) (end 137.16 114.808) (width 0.254) (layer F.Cu) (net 2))
 (segment (start 137.16 112.883303) (end 137.16 113.284) (width 0.254) (layer F.Cu) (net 2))
 (segment (start 136.704218 111.694273) (end 136.704218 112.427521) (width 0.254) (layer F.Cu) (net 2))
 (segment (start 136.704218 112.427521) (end 137.16 112.883303) (width 0.254) (layer F.Cu) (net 2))
 (segment (start 135.408619 110.398674) (end 136.704218 111.694273) (width 0.254) (layer F.Cu) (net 2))
 (segment (start 135.408619 109.474) (end 135.408619 110.398674) (width 0.254) (layer F.Cu) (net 2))
 (segment (start 133.604 118.896) (end 132.736 118.896) (width 0.254) (layer F.Cu) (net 3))
 (segment (start 132.736 118.896) (end 131.64 117.8) (width 0.254) (layer F.Cu) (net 3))
 (segment (start 133.604 118.896) (end 133.604 118.871) (width 0.254) (layer F.Cu) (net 3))
 (segment (start 132.025 117.8) (end 131.64 117.8) (width 0.254) (layer F.Cu) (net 3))
 (segment (start 136.398 118.396) (end 134.104 118.396) (width 0.254) (layer F.Cu) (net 3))
 (segment (start 134.104 118.396) (end 133.604 118.896) (width 0.254) (layer F.Cu) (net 3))
 (segment (start 136.761 117.348) (end 136.253 117.348) (width 0.254) (layer F.Cu) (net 4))
 (segment (start 136.253 117.348) (end 135.636 116.731) (width 0.254) (layer F.Cu) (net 4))
 (segment (start 138.309 118.896) (end 136.761 117.348) (width 0.254) (layer F.Cu) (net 4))
 (segment (start 137.308619 111.674) (end 137.308619 112.229697) (width 0.254) (layer F.Cu) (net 4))
 (segment (start 137.308619 112.229697) (end 137.689401 112.610479) (width 0.254) (layer F.Cu) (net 4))
 (segment (start 137.689401 112.610479) (end 137.689401 114.059479) (width 0.254) (layer F.Cu) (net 4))
 (segment (start 137.689401 114.059479) (end 137.839401 114.209479) (width 0.254) (layer F.Cu) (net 4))
 (segment (start 137.839401 114.209479) (end 137.839401 115.406521) (width 0.254) (layer F.Cu) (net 4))
 (segment (start 137.839401 115.406521) (end 137.783521 115.462401) (width 0.254) (layer F.Cu) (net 4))
 (segment (start 137.783521 115.462401) (end 136.490401 115.462401) (width 0.254) (layer F.Cu) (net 4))
 (segment (start 136.490401 115.462401) (end 135.836 114.808) (width 0.254) (layer F.Cu) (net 4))
 (segment (start 135.836 114.808) (end 135.636 114.808) (width 0.254) (layer F.Cu) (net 4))
 (segment (start 137.308619 111.674) (end 137.308619 111.879) (width 0.254) (layer F.Cu) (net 4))
 (segment (start 138.938 118.896) (end 138.309 118.896) (width 0.254) (layer F.Cu) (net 4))
 (segment (start 135.636 116.731) (end 135.636 115.312) (width 0.254) (layer F.Cu) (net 4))
 (segment (start 135.636 115.312) (end 135.636 114.808) (width 0.254) (layer F.Cu) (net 4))
 (segment (start 137.348 120.396) (end 137.438 120.396) (width 0.254) (layer F.Cu) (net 4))
 (segment (start 137.438 120.396) (end 138.938 118.896) (width 0.254) (layer F.Cu) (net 4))
 (segment (start 137.308619 111.512937) (end 138.548619 111.512937) (width 0.254) (layer F.Cu) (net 4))
 (segment (start 138.548619 111.512937) (end 138.898619 111.162937) (width 0.254) (layer F.Cu) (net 4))
 (segment (start 138.43 112.268) (end 138.137901 111.975901) (width 0.254) (layer B.Cu) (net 5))
 (segment (start 138.137901 111.975901) (end 138.124802 111.975901) (width 0.254) (layer B.Cu) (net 5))
 (segment (start 138.124802 111.975901) (end 137.668 111.519099) (width 0.254) (layer B.Cu) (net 5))
 (segment (start 138.66 113.284) (end 138.66 112.498) (width 0.254) (layer F.Cu) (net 5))
 (segment (start 138.66 112.498) (end 138.43 112.268) (width 0.254) (layer F.Cu) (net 5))
 (segment (start 137.668 110.49) (end 138.081091 110.49) (width 0.254) (layer F.Cu) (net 5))
 (segment (start 138.081091 110.49) (end 138.087555 110.483536) (width 0.254) (layer F.Cu) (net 5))
 (segment (start 138.087555 110.483536) (end 140.322464 110.483536) (width 0.254) (layer F.Cu) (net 5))
 (segment (start 140.322464 110.483536) (end 140.462 110.344) (width 0.254) (layer F.Cu) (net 5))
 (segment (start 140.462 110.344) (end 140.462 109.69) (width 0.254) (layer F.Cu) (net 5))
 (segment (start 137.668 110.49) (end 137.668 111.519099) (width 0.254) (layer B.Cu) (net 5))
 (via (at 138.43 112.268) (size 0.5842) (drill 0.381) (layers F.Cu B.Cu) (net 5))
 (segment (start 137.308619 109.474) (end 137.308619 110.130619) (width 0.254) (layer F.Cu) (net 5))
 (segment (start 137.308619 110.130619) (end 137.668 110.49) (width 0.254) (layer F.Cu) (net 5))
 (via (at 137.668 110.49) (size 0.5842) (drill 0.381) (layers F.Cu B.Cu) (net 5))
 (segment (start 134.330619 108.204) (end 136.822619 108.204) (width 0.254) (layer F.Cu) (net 5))
 (segment (start 136.822619 108.204) (end 137.308619 108.69) (width 0.254) (layer F.Cu) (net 5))
 (segment (start 137.308619 108.69) (end 137.308619 109.474) (width 0.254) (layer F.Cu) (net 5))
 (segment (start 133.818619 109.22) (end 133.818619 108.716) (width 0.254) (layer F.Cu) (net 5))
 (segment (start 133.818619 108.716) (end 134.330619 108.204) (width 0.254) (layer F.Cu) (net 5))
 (segment (start 140.462 111.29) (end 140.462 119.15) (width 0.254) (layer F.Cu) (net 6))
 (segment (start 135.408619 111.674) (end 135.408619 113.080619) (width 0.254) (layer F.Cu) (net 9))
 (segment (start 135.408619 113.080619) (end 135.636 113.308) (width 0.254) (layer F.Cu) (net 9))
 (segment (start 133.818619 110.72) (end 134.454619 110.72) (width 0.254) (layer F.Cu) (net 9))
 (segment (start 134.454619 110.72) (end 135.408619 111.674) (width 0.254) (layer F.Cu) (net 9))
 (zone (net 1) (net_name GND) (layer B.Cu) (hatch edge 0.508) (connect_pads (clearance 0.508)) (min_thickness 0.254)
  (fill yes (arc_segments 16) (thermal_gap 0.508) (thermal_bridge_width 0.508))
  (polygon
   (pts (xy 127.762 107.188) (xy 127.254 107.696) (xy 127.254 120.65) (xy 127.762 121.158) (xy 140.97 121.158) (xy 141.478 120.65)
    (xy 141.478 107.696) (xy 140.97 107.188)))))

